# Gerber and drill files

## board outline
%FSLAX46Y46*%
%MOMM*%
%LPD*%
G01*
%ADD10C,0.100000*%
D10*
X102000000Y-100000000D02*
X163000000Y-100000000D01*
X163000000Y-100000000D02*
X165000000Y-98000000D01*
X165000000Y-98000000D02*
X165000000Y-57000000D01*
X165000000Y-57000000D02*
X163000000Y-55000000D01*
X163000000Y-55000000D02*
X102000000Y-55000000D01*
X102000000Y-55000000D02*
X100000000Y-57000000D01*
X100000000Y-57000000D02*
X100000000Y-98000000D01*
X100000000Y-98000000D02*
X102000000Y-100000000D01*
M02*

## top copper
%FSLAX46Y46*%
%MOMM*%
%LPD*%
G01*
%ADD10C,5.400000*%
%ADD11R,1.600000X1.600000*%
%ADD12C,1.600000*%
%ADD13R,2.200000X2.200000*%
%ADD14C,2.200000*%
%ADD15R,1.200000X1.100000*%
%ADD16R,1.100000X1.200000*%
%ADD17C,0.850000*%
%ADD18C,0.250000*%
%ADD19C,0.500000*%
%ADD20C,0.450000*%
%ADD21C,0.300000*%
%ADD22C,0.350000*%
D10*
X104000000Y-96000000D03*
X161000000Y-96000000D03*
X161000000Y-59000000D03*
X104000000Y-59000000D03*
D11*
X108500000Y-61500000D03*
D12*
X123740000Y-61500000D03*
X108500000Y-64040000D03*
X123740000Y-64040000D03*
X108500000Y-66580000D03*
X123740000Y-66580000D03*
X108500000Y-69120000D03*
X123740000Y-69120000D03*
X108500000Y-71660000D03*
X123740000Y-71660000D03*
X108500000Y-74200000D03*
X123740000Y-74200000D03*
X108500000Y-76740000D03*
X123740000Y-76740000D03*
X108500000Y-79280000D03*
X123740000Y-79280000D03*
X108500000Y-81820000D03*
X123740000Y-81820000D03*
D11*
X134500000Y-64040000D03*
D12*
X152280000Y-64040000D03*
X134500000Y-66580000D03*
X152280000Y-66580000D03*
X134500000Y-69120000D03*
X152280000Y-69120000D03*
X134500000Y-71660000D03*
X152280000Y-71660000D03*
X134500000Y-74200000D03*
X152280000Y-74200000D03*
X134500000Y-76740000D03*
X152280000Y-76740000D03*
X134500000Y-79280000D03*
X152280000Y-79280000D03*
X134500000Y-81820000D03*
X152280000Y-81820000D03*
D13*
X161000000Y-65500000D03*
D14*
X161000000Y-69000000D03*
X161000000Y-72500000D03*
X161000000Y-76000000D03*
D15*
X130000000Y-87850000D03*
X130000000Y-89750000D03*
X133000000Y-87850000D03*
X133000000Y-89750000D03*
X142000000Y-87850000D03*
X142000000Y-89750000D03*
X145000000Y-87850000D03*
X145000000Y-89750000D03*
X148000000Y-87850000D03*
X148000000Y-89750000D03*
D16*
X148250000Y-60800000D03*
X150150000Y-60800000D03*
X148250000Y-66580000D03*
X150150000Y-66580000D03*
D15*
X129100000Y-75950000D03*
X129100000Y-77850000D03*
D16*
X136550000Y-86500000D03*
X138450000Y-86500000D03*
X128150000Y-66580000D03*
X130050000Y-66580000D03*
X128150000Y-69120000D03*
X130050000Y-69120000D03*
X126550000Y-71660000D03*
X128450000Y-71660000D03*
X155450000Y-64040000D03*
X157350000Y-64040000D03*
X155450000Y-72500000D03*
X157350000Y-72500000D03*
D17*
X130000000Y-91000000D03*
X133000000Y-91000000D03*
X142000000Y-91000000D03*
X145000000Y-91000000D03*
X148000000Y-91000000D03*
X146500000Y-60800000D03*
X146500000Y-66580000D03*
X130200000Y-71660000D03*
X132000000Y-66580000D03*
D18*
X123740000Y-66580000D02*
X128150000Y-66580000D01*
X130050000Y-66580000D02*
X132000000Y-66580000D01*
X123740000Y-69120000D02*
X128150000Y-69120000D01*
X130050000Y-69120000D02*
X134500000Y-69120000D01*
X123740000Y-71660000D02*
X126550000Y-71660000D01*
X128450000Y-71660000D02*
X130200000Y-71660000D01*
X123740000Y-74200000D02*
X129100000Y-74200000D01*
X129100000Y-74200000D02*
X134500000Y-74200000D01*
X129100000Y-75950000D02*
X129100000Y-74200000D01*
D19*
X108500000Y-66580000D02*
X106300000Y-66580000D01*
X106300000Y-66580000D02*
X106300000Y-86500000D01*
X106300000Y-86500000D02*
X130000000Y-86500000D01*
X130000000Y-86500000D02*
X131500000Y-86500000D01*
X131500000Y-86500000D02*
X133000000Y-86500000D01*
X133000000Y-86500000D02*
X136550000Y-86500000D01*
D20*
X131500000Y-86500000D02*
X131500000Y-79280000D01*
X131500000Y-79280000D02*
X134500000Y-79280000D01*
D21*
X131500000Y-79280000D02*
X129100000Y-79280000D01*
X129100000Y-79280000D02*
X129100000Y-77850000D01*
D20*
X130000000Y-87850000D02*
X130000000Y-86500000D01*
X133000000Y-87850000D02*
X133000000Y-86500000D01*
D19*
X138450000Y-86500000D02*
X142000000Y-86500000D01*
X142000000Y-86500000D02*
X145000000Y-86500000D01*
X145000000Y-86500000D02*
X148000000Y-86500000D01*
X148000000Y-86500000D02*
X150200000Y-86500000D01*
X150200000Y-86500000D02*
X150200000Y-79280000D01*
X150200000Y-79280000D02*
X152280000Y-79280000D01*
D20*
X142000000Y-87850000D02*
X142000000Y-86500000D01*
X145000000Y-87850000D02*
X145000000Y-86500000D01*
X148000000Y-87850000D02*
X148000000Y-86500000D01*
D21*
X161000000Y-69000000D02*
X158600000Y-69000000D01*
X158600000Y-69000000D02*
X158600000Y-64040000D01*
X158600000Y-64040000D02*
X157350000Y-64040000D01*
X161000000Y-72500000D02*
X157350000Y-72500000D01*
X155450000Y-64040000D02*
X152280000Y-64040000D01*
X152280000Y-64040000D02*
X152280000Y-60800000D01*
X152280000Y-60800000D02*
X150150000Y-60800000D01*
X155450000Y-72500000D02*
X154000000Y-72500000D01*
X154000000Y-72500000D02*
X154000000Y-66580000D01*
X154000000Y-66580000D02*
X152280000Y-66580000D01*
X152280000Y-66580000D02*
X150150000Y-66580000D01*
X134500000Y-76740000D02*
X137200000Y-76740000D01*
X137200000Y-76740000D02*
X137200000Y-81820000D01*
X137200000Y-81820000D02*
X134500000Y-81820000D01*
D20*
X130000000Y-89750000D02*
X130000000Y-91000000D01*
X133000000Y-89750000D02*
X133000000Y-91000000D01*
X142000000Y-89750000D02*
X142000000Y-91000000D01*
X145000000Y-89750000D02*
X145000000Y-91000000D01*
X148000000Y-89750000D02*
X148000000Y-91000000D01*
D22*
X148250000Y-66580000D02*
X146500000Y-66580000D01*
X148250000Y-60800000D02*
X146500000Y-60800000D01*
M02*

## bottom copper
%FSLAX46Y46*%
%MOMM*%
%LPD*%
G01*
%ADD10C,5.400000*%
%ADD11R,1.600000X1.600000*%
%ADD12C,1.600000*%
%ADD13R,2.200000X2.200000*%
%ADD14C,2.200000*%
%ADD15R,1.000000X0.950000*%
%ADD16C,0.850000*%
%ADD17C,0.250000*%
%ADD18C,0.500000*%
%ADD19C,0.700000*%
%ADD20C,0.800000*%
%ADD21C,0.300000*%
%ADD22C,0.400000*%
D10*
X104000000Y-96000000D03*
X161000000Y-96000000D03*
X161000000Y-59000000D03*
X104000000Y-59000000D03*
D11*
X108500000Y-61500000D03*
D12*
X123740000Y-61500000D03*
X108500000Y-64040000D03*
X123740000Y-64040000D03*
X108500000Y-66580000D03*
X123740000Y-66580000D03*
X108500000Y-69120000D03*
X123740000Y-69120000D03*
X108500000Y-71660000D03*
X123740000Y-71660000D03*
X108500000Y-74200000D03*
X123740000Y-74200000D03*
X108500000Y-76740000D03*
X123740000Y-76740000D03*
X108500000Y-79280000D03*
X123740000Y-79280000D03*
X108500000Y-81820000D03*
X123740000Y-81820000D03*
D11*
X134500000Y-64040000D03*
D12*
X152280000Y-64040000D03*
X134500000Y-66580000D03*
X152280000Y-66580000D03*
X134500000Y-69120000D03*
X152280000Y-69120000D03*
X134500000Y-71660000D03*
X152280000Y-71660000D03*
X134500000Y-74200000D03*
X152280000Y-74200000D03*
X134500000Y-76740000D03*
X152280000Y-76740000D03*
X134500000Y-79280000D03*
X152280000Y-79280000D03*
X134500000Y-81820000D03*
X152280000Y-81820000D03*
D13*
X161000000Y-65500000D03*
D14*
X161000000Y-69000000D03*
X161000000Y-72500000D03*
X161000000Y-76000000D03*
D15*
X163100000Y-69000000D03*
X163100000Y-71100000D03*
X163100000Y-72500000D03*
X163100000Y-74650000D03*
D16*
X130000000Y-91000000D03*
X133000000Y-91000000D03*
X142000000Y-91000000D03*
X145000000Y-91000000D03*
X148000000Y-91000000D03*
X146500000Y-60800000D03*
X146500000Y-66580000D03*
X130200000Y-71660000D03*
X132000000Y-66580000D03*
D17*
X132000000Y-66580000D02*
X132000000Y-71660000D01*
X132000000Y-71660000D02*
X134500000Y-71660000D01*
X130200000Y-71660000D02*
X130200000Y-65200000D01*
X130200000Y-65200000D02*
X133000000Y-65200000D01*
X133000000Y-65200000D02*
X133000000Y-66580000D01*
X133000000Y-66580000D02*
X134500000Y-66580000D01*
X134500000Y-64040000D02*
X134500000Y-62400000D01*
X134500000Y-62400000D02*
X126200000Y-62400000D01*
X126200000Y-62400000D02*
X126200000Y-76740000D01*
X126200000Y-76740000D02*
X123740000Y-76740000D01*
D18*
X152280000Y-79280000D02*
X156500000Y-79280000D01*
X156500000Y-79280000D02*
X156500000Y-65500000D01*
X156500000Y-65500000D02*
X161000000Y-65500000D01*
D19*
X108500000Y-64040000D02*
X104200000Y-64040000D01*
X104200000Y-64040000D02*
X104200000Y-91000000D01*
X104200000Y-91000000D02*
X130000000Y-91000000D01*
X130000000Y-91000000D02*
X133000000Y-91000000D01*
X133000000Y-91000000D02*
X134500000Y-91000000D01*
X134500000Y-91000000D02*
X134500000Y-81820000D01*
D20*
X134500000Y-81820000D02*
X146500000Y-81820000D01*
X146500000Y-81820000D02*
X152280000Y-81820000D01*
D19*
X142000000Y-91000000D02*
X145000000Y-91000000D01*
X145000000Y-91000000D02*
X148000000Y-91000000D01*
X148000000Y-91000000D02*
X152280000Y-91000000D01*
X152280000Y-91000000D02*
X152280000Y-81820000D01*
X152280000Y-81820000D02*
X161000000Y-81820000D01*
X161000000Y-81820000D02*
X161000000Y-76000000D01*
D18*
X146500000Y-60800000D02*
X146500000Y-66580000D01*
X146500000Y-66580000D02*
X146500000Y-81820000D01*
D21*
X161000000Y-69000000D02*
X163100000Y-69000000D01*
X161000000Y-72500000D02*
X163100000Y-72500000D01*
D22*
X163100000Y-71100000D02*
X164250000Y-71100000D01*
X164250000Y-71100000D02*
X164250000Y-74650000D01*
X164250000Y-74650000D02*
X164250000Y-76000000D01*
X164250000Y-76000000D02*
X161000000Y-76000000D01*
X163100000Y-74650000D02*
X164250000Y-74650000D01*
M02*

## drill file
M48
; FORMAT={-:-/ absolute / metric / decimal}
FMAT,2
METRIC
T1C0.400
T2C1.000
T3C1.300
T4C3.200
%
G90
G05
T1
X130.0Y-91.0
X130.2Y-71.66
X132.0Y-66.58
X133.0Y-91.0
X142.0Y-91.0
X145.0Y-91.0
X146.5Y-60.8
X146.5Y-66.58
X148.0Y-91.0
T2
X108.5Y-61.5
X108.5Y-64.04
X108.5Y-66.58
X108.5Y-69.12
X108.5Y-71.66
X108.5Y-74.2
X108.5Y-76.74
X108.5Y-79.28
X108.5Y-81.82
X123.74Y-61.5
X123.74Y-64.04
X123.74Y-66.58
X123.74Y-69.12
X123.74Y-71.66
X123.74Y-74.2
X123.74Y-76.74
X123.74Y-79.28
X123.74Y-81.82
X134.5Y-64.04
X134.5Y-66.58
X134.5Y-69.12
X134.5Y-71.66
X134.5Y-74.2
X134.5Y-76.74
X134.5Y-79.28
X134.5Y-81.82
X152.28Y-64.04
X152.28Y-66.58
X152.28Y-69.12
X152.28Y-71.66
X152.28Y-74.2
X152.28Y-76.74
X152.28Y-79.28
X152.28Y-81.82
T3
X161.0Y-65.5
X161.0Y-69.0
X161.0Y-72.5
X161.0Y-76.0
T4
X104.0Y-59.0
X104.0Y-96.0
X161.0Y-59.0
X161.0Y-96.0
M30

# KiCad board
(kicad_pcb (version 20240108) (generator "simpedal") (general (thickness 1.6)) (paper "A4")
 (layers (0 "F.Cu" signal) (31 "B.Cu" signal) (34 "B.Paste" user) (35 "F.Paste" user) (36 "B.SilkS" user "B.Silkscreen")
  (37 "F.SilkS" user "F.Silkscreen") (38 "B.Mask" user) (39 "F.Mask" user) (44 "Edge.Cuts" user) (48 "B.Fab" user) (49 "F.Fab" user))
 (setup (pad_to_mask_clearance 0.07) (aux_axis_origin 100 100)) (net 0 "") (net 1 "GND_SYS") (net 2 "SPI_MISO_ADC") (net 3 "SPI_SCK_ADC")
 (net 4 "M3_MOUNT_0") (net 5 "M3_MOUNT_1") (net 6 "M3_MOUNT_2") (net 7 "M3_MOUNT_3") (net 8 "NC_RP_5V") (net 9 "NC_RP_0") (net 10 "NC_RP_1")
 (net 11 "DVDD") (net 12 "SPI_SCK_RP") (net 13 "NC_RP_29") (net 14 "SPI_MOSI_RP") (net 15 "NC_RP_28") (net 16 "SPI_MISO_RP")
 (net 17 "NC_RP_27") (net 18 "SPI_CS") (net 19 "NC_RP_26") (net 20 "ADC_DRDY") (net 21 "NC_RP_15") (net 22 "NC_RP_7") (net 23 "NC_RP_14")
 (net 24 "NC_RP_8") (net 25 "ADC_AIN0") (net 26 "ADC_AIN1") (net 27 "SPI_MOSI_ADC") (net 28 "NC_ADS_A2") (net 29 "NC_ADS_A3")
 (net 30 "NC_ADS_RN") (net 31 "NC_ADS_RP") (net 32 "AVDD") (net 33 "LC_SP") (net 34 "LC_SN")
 (via (at 130.0000 91.0000) (size 0.85) (drill 0.4) (layers "F.Cu" "B.Cu") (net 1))
 (via (at 133.0000 91.0000) (size 0.85) (drill 0.4) (layers "F.Cu" "B.Cu") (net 1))
 (via (at 142.0000 91.0000) (size 0.85) (drill 0.4) (layers "F.Cu" "B.Cu") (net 1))
 (via (at 145.0000 91.0000) (size 0.85) (drill 0.4) (layers "F.Cu" "B.Cu") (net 1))
 (via (at 148.0000 91.0000) (size 0.85) (drill 0.4) (layers "F.Cu" "B.Cu") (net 1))
 (via (at 146.5000 60.8000) (size 0.85) (drill 0.4) (layers "F.Cu" "B.Cu") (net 1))
 (via (at 146.5000 66.5800) (size 0.85) (drill 0.4) (layers "F.Cu" "B.Cu") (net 1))
 (via (at 130.2000 71.6600) (size 0.85) (drill 0.4) (layers "F.Cu" "B.Cu") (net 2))
 (via (at 132.0000 66.5800) (size 0.85) (drill 0.4) (layers "F.Cu" "B.Cu") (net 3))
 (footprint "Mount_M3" (layer "F.Cu") (at 104.0000 96.0000)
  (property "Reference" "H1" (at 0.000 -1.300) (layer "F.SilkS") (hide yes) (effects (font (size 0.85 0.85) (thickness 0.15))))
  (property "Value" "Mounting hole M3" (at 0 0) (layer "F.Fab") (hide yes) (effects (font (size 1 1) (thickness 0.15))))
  (pad "1" thru_hole circle (at 0.0000 0.0000) (size 5.4 5.4) (drill 3.2) (layers "*.Cu" "*.Mask") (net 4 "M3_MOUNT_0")))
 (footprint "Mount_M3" (layer "F.Cu") (at 161.0000 96.0000)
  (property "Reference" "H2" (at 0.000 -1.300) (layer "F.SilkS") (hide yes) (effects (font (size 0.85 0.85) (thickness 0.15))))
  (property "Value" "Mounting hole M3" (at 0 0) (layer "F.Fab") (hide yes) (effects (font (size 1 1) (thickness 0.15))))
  (pad "1" thru_hole circle (at 0.0000 0.0000) (size 5.4 5.4) (drill 3.2) (layers "*.Cu" "*.Mask") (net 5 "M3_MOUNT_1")))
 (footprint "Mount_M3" (layer "F.Cu") (at 161.0000 59.0000)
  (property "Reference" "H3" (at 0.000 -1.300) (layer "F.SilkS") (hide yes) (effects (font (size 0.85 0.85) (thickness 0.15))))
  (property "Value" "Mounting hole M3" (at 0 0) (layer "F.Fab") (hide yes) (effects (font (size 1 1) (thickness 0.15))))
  (pad "1" thru_hole circle (at 0.0000 0.0000) (size 5.4 5.4) (drill 3.2) (layers "*.Cu" "*.Mask") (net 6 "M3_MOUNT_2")))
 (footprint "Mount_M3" (layer "F.Cu") (at 104.0000 59.0000)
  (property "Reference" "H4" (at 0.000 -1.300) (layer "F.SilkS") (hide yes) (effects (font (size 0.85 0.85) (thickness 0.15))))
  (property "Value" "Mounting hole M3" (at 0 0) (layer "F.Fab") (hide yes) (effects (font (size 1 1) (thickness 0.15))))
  (pad "1" thru_hole circle (at 0.0000 0.0000) (size 5.4 5.4) (drill 3.2) (layers "*.Cu" "*.Mask") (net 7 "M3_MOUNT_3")))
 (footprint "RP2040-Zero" (layer "F.Cu") (at 116.1200 71.6600)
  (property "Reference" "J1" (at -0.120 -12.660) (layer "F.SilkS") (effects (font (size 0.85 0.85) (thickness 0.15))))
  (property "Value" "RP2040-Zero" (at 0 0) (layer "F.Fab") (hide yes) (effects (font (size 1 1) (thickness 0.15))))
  (pad "1" thru_hole rect (at -7.6200 -10.1600) (size 1.6 1.6) (drill 1) (layers "*.Cu" "*.Mask") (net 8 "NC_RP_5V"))
  (pad "2" thru_hole circle (at 7.6200 -10.1600) (size 1.6 1.6) (drill 1) (layers "*.Cu" "*.Mask") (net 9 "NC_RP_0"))
  (pad "3" thru_hole circle (at -7.6200 -7.6200) (size 1.6 1.6) (drill 1) (layers "*.Cu" "*.Mask") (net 1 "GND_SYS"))
  (pad "4" thru_hole circle (at 7.6200 -7.6200) (size 1.6 1.6) (drill 1) (layers "*.Cu" "*.Mask") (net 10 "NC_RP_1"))
  (pad "5" thru_hole circle (at -7.6200 -5.0800) (size 1.6 1.6) (drill 1) (layers "*.Cu" "*.Mask") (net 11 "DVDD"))
  (pad "6" thru_hole circle (at 7.6200 -5.0800) (size 1.6 1.6) (drill 1) (layers "*.Cu" "*.Mask") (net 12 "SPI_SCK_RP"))
  (pad "7" thru_hole circle (at -7.6200 -2.5400) (size 1.6 1.6) (drill 1) (layers "*.Cu" "*.Mask") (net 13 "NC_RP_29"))
  (pad "8" thru_hole circle (at 7.6200 -2.5400) (size 1.6 1.6) (drill 1) (layers "*.Cu" "*.Mask") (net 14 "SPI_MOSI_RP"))
  (pad "9" thru_hole circle (at -7.6200 0.0000) (size 1.6 1.6) (drill 1) (layers "*.Cu" "*.Mask") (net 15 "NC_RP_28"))
  (pad "10" thru_hole circle (at 7.6200 0.0000) (size 1.6 1.6) (drill 1) (layers "*.Cu" "*.Mask") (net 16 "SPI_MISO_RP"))
  (pad "11" thru_hole circle (at -7.6200 2.5400) (size 1.6 1.6) (drill 1) (layers "*.Cu" "*.Mask") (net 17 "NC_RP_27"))
  (pad "12" thru_hole circle (at 7.6200 2.5400) (size 1.6 1.6) (drill 1) (layers "*.Cu" "*.Mask") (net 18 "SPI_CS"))
  (pad "13" thru_hole circle (at -7.6200 5.0800) (size 1.6 1.6) (drill 1) (layers "*.Cu" "*.Mask") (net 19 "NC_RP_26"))
  (pad "14" thru_hole circle (at 7.6200 5.0800) (size 1.6 1.6) (drill 1) (layers "*.Cu" "*.Mask") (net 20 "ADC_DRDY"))
  (pad "15" thru_hole circle (at -7.6200 7.6200) (size 1.6 1.6) (drill 1) (layers "*.Cu" "*.Mask") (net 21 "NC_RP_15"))
  (pad "16" thru_hole circle (at 7.6200 7.6200) (size 1.6 1.6) (drill 1) (layers "*.Cu" "*.Mask") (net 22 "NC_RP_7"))
  (pad "17" thru_hole circle (at -7.6200 10.1600) (size 1.6 1.6) (drill 1) (layers "*.Cu" "*.Mask") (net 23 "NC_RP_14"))
  (pad "18" thru_hole circle (at 7.6200 10.1600) (size 1.6 1.6) (drill 1) (layers "*.Cu" "*.Mask") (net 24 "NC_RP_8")))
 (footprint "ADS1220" (layer "F.Cu") (at 143.3900 72.9300)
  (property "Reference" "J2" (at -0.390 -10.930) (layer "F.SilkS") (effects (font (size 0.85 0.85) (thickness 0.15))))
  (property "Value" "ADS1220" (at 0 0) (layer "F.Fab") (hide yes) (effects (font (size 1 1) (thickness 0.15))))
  (pad "1" thru_hole rect (at -8.8900 -8.8900) (size 1.6 1.6) (drill 1) (layers "*.Cu" "*.Mask") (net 20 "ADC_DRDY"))
  (pad "2" thru_hole circle (at 8.8900 -8.8900) (size 1.6 1.6) (drill 1) (layers "*.Cu" "*.Mask") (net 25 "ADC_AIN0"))
  (pad "3" thru_hole circle (at -8.8900 -6.3500) (size 1.6 1.6) (drill 1) (layers "*.Cu" "*.Mask") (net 2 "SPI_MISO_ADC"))
  (pad "4" thru_hole circle (at 8.8900 -6.3500) (size 1.6 1.6) (drill 1) (layers "*.Cu" "*.Mask") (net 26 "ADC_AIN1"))
  (pad "5" thru_hole circle (at -8.8900 -3.8100) (size 1.6 1.6) (drill 1) (layers "*.Cu" "*.Mask") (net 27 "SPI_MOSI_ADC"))
  (pad "6" thru_hole circle (at 8.8900 -3.8100) (size 1.6 1.6) (drill 1) (layers "*.Cu" "*.Mask") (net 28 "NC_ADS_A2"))
  (pad "7" thru_hole circle (at -8.8900 -1.2700) (size 1.6 1.6) (drill 1) (layers "*.Cu" "*.Mask") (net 3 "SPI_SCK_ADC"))
  (pad "8" thru_hole circle (at 8.8900 -1.2700) (size 1.6 1.6) (drill 1) (layers "*.Cu" "*.Mask") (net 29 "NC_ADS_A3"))
  (pad "9" thru_hole circle (at -8.8900 1.2700) (size 1.6 1.6) (drill 1) (layers "*.Cu" "*.Mask") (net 18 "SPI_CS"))
  (pad "10" thru_hole circle (at 8.8900 1.2700) (size 1.6 1.6) (drill 1) (layers "*.Cu" "*.Mask") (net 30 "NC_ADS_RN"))
  (pad "11" thru_hole circle (at -8.8900 3.8100) (size 1.6 1.6) (drill 1) (layers "*.Cu" "*.Mask") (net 1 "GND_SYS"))
  (pad "12" thru_hole circle (at 8.8900 3.8100) (size 1.6 1.6) (drill 1) (layers "*.Cu" "*.Mask") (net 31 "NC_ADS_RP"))
  (pad "13" thru_hole circle (at -8.8900 6.3500) (size 1.6 1.6) (drill 1) (layers "*.Cu" "*.Mask") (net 11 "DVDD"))
  (pad "14" thru_hole circle (at 8.8900 6.3500) (size 1.6 1.6) (drill 1) (layers "*.Cu" "*.Mask") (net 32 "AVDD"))
  (pad "15" thru_hole circle (at -8.8900 8.8900) (size 1.6 1.6) (drill 1) (layers "*.Cu" "*.Mask") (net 1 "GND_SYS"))
  (pad "16" thru_hole circle (at 8.8900 8.8900) (size 1.6 1.6) (drill 1) (layers "*.Cu" "*.Mask") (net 1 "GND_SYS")))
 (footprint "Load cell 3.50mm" (layer "F.Cu") (at 161.0000 70.7500)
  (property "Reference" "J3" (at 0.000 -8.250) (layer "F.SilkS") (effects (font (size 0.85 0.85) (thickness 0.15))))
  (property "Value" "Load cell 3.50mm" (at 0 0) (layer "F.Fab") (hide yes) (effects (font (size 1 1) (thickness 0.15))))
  (pad "1" thru_hole rect (at 0.0000 -5.2500) (size 2.2 2.2) (drill 1.3) (layers "*.Cu" "*.Mask") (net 32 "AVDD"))
  (pad "2" thru_hole circle (at 0.0000 -1.7500) (size 2.2 2.2) (drill 1.3) (layers "*.Cu" "*.Mask") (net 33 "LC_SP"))
  (pad "3" thru_hole circle (at 0.0000 1.7500) (size 2.2 2.2) (drill 1.3) (layers "*.Cu" "*.Mask") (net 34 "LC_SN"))
  (pad "4" thru_hole circle (at 0.0000 5.2500) (size 2.2 2.2) (drill 1.3) (layers "*.Cu" "*.Mask") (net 1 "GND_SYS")))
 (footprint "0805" (layer "F.Cu") (at 130.0000 88.8000)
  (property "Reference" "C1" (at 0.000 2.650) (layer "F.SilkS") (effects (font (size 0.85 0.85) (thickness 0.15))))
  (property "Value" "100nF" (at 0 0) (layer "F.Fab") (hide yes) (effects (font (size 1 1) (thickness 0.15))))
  (pad "2" smd rect (at 0.0000 -0.9500) (size 1.2 1.1) (layers "F.Cu" "F.Paste" "F.Mask") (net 11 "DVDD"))
  (pad "1" smd rect (at 0.0000 0.9500) (size 1.2 1.1) (layers "F.Cu" "F.Paste" "F.Mask") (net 1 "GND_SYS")))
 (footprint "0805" (layer "F.Cu") (at 133.0000 88.8000)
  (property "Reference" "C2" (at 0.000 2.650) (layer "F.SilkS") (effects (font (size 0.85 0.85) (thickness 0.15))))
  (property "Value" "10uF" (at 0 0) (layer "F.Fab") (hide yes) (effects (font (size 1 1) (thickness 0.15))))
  (pad "2" smd rect (at 0.0000 -0.9500) (size 1.2 1.1) (layers "F.Cu" "F.Paste" "F.Mask") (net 11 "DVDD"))
  (pad "1" smd rect (at 0.0000 0.9500) (size 1.2 1.1) (layers "F.Cu" "F.Paste" "F.Mask") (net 1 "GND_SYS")))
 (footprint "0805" (layer "F.Cu") (at 142.0000 88.8000)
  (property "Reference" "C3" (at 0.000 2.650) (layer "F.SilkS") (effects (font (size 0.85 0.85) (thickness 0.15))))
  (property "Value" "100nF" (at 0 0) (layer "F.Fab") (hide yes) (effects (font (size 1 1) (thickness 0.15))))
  (pad "2" smd rect (at 0.0000 -0.9500) (size 1.2 1.1) (layers "F.Cu" "F.Paste" "F.Mask") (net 32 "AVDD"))
  (pad "1" smd rect (at 0.0000 0.9500) (size 1.2 1.1) (layers "F.Cu" "F.Paste" "F.Mask") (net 1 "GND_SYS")))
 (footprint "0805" (layer "F.Cu") (at 145.0000 88.8000)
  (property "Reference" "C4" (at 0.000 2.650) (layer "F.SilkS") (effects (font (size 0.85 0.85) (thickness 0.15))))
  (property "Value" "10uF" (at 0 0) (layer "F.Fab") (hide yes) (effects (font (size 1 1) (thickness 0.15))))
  (pad "2" smd rect (at 0.0000 -0.9500) (size 1.2 1.1) (layers "F.Cu" "F.Paste" "F.Mask") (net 32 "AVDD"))
  (pad "1" smd rect (at 0.0000 0.9500) (size 1.2 1.1) (layers "F.Cu" "F.Paste" "F.Mask") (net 1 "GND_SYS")))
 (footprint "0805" (layer "F.Cu") (at 148.0000 88.8000)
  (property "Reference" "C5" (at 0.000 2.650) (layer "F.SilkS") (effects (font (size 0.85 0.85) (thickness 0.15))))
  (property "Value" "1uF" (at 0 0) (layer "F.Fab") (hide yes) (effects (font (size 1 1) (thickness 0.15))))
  (pad "2" smd rect (at 0.0000 -0.9500) (size 1.2 1.1) (layers "F.Cu" "F.Paste" "F.Mask") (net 32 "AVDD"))
  (pad "1" smd rect (at 0.0000 0.9500) (size 1.2 1.1) (layers "F.Cu" "F.Paste" "F.Mask") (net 1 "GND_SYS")))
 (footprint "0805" (layer "F.Cu") (at 149.2000 60.8000)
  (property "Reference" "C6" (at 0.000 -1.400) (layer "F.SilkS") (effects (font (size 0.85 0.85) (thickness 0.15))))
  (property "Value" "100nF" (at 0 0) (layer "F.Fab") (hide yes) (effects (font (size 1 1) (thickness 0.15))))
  (pad "1" smd rect (at -0.9500 0.0000) (size 1.1 1.2) (layers "F.Cu" "F.Paste" "F.Mask") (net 1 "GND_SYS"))
  (pad "2" smd rect (at 0.9500 0.0000) (size 1.1 1.2) (layers "F.Cu" "F.Paste" "F.Mask") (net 25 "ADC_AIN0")))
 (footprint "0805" (layer "F.Cu") (at 149.2000 66.5800)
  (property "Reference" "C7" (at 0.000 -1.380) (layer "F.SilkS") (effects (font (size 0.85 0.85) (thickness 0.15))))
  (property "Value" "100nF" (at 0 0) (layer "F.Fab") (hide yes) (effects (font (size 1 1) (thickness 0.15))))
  (pad "1" smd rect (at -0.9500 0.0000) (size 1.1 1.2) (layers "F.Cu" "F.Paste" "F.Mask") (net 1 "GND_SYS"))
  (pad "2" smd rect (at 0.9500 0.0000) (size 1.1 1.2) (layers "F.Cu" "F.Paste" "F.Mask") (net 26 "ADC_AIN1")))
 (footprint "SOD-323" (layer "B.Cu") (at 163.1000 70.0500)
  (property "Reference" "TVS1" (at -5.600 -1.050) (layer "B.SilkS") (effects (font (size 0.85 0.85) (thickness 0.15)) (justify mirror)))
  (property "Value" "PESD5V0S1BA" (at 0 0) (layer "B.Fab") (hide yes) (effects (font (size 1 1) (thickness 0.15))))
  (pad "1" smd rect (at 0.0000 -1.0500) (size 1 0.95) (layers "B.Cu" "B.Paste" "B.Mask") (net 33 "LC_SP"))
  (pad "2" smd rect (at 0.0000 1.0500) (size 1 0.95) (layers "B.Cu" "B.Paste" "B.Mask") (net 1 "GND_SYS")))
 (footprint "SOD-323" (layer "B.Cu") (at 163.1000 73.5750)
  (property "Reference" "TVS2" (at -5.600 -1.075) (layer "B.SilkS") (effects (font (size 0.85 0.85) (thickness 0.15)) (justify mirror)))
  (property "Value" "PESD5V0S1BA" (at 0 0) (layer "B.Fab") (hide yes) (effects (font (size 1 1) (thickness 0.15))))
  (pad "1" smd rect (at 0.0000 -1.0750) (size 1 0.95) (layers "B.Cu" "B.Paste" "B.Mask") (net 34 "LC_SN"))
  (pad "2" smd rect (at 0.0000 1.0750) (size 1 0.95) (layers "B.Cu" "B.Paste" "B.Mask") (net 1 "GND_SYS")))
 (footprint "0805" (layer "F.Cu") (at 129.1000 76.9000)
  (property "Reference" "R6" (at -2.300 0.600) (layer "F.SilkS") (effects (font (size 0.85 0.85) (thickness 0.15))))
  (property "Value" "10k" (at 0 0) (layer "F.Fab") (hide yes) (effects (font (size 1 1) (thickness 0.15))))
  (pad "2" smd rect (at 0.0000 -0.9500) (size 1.2 1.1) (layers "F.Cu" "F.Paste" "F.Mask") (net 18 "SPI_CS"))
  (pad "1" smd rect (at 0.0000 0.9500) (size 1.2 1.1) (layers "F.Cu" "F.Paste" "F.Mask") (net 11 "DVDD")))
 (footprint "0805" (layer "F.Cu") (at 137.5000 86.5000)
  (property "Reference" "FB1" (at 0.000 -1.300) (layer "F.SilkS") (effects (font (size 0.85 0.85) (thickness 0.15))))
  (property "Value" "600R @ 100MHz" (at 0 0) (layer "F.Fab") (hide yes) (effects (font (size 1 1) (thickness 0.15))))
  (pad "1" smd rect (at -0.9500 0.0000) (size 1.1 1.2) (layers "F.Cu" "F.Paste" "F.Mask") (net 11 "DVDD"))
  (pad "2" smd rect (at 0.9500 0.0000) (size 1.1 1.2) (layers "F.Cu" "F.Paste" "F.Mask") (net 32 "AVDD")))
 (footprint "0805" (layer "F.Cu") (at 129.1000 66.5800)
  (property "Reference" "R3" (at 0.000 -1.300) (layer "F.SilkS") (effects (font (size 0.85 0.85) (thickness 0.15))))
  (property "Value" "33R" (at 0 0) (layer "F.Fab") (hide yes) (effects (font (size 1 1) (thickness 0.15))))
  (pad "1" smd rect (at -0.9500 0.0000) (size 1.1 1.2) (layers "F.Cu" "F.Paste" "F.Mask") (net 12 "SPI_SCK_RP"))
  (pad "2" smd rect (at 0.9500 0.0000) (size 1.1 1.2) (layers "F.Cu" "F.Paste" "F.Mask") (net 3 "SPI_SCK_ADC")))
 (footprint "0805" (layer "F.Cu") (at 129.1000 69.1200)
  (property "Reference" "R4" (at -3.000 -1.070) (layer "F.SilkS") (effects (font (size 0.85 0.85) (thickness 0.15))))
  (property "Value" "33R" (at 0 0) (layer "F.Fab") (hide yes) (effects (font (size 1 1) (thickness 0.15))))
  (pad "1" smd rect (at -0.9500 0.0000) (size 1.1 1.2) (layers "F.Cu" "F.Paste" "F.Mask") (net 14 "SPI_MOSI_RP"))
  (pad "2" smd rect (at 0.9500 0.0000) (size 1.1 1.2) (layers "F.Cu" "F.Paste" "F.Mask") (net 27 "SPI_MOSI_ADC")))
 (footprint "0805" (layer "F.Cu") (at 127.5000 71.6600)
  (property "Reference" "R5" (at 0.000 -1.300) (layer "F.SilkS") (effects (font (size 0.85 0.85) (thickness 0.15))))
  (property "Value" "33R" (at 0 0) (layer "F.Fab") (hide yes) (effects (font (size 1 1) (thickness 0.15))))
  (pad "1" smd rect (at -0.9500 0.0000) (size 1.1 1.2) (layers "F.Cu" "F.Paste" "F.Mask") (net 16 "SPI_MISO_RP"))
  (pad "2" smd rect (at 0.9500 0.0000) (size 1.1 1.2) (layers "F.Cu" "F.Paste" "F.Mask") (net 2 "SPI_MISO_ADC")))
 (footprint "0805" (layer "F.Cu") (at 156.4000 64.0400)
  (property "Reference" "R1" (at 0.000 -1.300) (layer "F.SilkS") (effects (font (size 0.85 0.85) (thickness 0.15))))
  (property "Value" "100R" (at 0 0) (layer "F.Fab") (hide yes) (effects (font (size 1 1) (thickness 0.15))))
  (pad "1" smd rect (at -0.9500 0.0000) (size 1.1 1.2) (layers "F.Cu" "F.Paste" "F.Mask") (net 25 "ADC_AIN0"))
  (pad "2" smd rect (at 0.9500 0.0000) (size 1.1 1.2) (layers "F.Cu" "F.Paste" "F.Mask") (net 33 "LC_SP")))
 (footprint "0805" (layer "F.Cu") (at 156.4000 72.5000)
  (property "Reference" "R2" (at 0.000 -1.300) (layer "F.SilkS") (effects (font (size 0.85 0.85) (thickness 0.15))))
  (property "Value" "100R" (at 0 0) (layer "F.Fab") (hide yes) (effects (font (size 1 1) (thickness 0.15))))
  (pad "1" smd rect (at -0.9500 0.0000) (size 1.1 1.2) (layers "F.Cu" "F.Paste" "F.Mask") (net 26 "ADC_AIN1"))
  (pad "2" smd rect (at 0.9500 0.0000) (size 1.1 1.2) (layers "F.Cu" "F.Paste" "F.Mask") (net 34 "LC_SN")))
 (segment (start 123.7400 66.5800) (end 128.1500 66.5800) (width 0.25) (layer "F.Cu") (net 12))
 (segment (start 130.0500 66.5800) (end 132.0000 66.5800) (width 0.25) (layer "F.Cu") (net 3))
 (segment (start 132.0000 66.5800) (end 132.0000 71.6600) (width 0.25) (layer "B.Cu") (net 3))
 (segment (start 132.0000 71.6600) (end 134.5000 71.6600) (width 0.25) (layer "B.Cu") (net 3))
 (segment (start 123.7400 69.1200) (end 128.1500 69.1200) (width 0.25) (layer "F.Cu") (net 14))
 (segment (start 130.0500 69.1200) (end 134.5000 69.1200) (width 0.25) (layer "F.Cu") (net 27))
 (segment (start 123.7400 71.6600) (end 126.5500 71.6600) (width 0.25) (layer "F.Cu") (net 16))
 (segment (start 128.4500 71.6600) (end 130.2000 71.6600) (width 0.25) (layer "F.Cu") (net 2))
 (segment (start 130.2000 71.6600) (end 130.2000 65.2000) (width 0.25) (layer "B.Cu") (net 2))
 (segment (start 130.2000 65.2000) (end 133.0000 65.2000) (width 0.25) (layer "B.Cu") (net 2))
 (segment (start 133.0000 65.2000) (end 133.0000 66.5800) (width 0.25) (layer "B.Cu") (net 2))
 (segment (start 133.0000 66.5800) (end 134.5000 66.5800) (width 0.25) (layer "B.Cu") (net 2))
 (segment (start 123.7400 74.2000) (end 129.1000 74.2000) (width 0.25) (layer "F.Cu") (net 18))
 (segment (start 129.1000 74.2000) (end 134.5000 74.2000) (width 0.25) (layer "F.Cu") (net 18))
 (segment (start 129.1000 75.9500) (end 129.1000 74.2000) (width 0.25) (layer "F.Cu") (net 18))
 (segment (start 134.5000 64.0400) (end 134.5000 62.4000) (width 0.25) (layer "B.Cu") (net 20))
 (segment (start 134.5000 62.4000) (end 126.2000 62.4000) (width 0.25) (layer "B.Cu") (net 20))
 (segment (start 126.2000 62.4000) (end 126.2000 76.7400) (width 0.25) (layer "B.Cu") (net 20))
 (segment (start 126.2000 76.7400) (end 123.7400 76.7400) (width 0.25) (layer "B.Cu") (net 20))
 (segment (start 108.5000 66.5800) (end 106.3000 66.5800) (width 0.5) (layer "F.Cu") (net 11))
 (segment (start 106.3000 66.5800) (end 106.3000 86.5000) (width 0.5) (layer "F.Cu") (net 11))
 (segment (start 106.3000 86.5000) (end 130.0000 86.5000) (width 0.5) (layer "F.Cu") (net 11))
 (segment (start 130.0000 86.5000) (end 131.5000 86.5000) (width 0.5) (layer "F.Cu") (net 11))
 (segment (start 131.5000 86.5000) (end 133.0000 86.5000) (width 0.5) (layer "F.Cu") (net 11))
 (segment (start 133.0000 86.5000) (end 136.5500 86.5000) (width 0.5) (layer "F.Cu") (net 11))
 (segment (start 131.5000 86.5000) (end 131.5000 79.2800) (width 0.45) (layer "F.Cu") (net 11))
 (segment (start 131.5000 79.2800) (end 134.5000 79.2800) (width 0.45) (layer "F.Cu") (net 11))
 (segment (start 131.5000 79.2800) (end 129.1000 79.2800) (width 0.3) (layer "F.Cu") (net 11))
 (segment (start 129.1000 79.2800) (end 129.1000 77.8500) (width 0.3) (layer "F.Cu") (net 11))
 (segment (start 130.0000 87.8500) (end 130.0000 86.5000) (width 0.45) (layer "F.Cu") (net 11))
 (segment (start 133.0000 87.8500) (end 133.0000 86.5000) (width 0.45) (layer "F.Cu") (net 11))
 (segment (start 138.4500 86.5000) (end 142.0000 86.5000) (width 0.5) (layer "F.Cu") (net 32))
 (segment (start 142.0000 86.5000) (end 145.0000 86.5000) (width 0.5) (layer "F.Cu") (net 32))
 (segment (start 145.0000 86.5000) (end 148.0000 86.5000) (width 0.5) (layer "F.Cu") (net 32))
 (segment (start 148.0000 86.5000) (end 150.2000 86.5000) (width 0.5) (layer "F.Cu") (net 32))
 (segment (start 150.2000 86.5000) (end 150.2000 79.2800) (width 0.5) (layer "F.Cu") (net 32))
 (segment (start 150.2000 79.2800) (end 152.2800 79.2800) (width 0.5) (layer "F.Cu") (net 32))
 (segment (start 142.0000 87.8500) (end 142.0000 86.5000) (width 0.45) (layer "F.Cu") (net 32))
 (segment (start 145.0000 87.8500) (end 145.0000 86.5000) (width 0.45) (layer "F.Cu") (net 32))
 (segment (start 148.0000 87.8500) (end 148.0000 86.5000) (width 0.45) (layer "F.Cu") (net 32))
 (segment (start 152.2800 79.2800) (end 156.5000 79.2800) (width 0.5) (layer "B.Cu") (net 32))
 (segment (start 156.5000 79.2800) (end 156.5000 65.5000) (width 0.5) (layer "B.Cu") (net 32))
 (segment (start 156.5000 65.5000) (end 161.0000 65.5000) (width 0.5) (layer "B.Cu") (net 32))
 (segment (start 161.0000 69.0000) (end 158.6000 69.0000) (width 0.3) (layer "F.Cu") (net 33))
 (segment (start 158.6000 69.0000) (end 158.6000 64.0400) (width 0.3) (layer "F.Cu") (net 33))
 (segment (start 158.6000 64.0400) (end 157.3500 64.0400) (width 0.3) (layer "F.Cu") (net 33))
 (segment (start 161.0000 72.5000) (end 157.3500 72.5000) (width 0.3) (layer "F.Cu") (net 34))
 (segment (start 155.4500 64.0400) (end 152.2800 64.0400) (width 0.3) (layer "F.Cu") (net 25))
 (segment (start 152.2800 64.0400) (end 152.2800 60.8000) (width 0.3) (layer "F.Cu") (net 25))
 (segment (start 152.2800 60.8000) (end 150.1500 60.8000) (width 0.3) (layer "F.Cu") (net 25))
 (segment (start 155.4500 72.5000) (end 154.0000 72.5000) (width 0.3) (layer "F.Cu") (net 26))
 (segment (start 154.0000 72.5000) (end 154.0000 66.5800) (width 0.3) (layer "F.Cu") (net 26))
 (segment (start 154.0000 66.5800) (end 152.2800 66.5800) (width 0.3) (layer "F.Cu") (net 26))
 (segment (start 152.2800 66.5800) (end 150.1500 66.5800) (width 0.3) (layer "F.Cu") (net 26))
 (segment (start 108.5000 64.0400) (end 104.2000 64.0400) (width 0.7) (layer "B.Cu") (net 1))
 (segment (start 104.2000 64.0400) (end 104.2000 91.0000) (width 0.7) (layer "B.Cu") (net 1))
 (segment (start 104.2000 91.0000) (end 130.0000 91.0000) (width 0.7) (layer "B.Cu") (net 1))
 (segment (start 130.0000 91.0000) (end 133.0000 91.0000) (width 0.7) (layer "B.Cu") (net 1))
 (segment (start 133.0000 91.0000) (end 134.5000 91.0000) (width 0.7) (layer "B.Cu") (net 1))
 (segment (start 134.5000 91.0000) (end 134.5000 81.8200) (width 0.7) (layer "B.Cu") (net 1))
 (segment (start 134.5000 76.7400) (end 137.2000 76.7400) (width 0.3) (layer "F.Cu") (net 1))
 (segment (start 137.2000 76.7400) (end 137.2000 81.8200) (width 0.3) (layer "F.Cu") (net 1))
 (segment (start 137.2000 81.8200) (end 134.5000 81.8200) (width 0.3) (layer "F.Cu") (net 1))
 (segment (start 134.5000 81.8200) (end 146.5000 81.8200) (width 0.8) (layer "B.Cu") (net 1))
 (segment (start 146.5000 81.8200) (end 152.2800 81.8200) (width 0.8) (layer "B.Cu") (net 1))
 (segment (start 142.0000 91.0000) (end 145.0000 91.0000) (width 0.7) (layer "B.Cu") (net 1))
 (segment (start 145.0000 91.0000) (end 148.0000 91.0000) (width 0.7) (layer "B.Cu") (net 1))
 (segment (start 148.0000 91.0000) (end 152.2800 91.0000) (width 0.7) (layer "B.Cu") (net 1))
 (segment (start 152.2800 91.0000) (end 152.2800 81.8200) (width 0.7) (layer "B.Cu") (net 1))
 (segment (start 152.2800 81.8200) (end 161.0000 81.8200) (width 0.7) (layer "B.Cu") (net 1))
 (segment (start 161.0000 81.8200) (end 161.0000 76.0000) (width 0.7) (layer "B.Cu") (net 1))
 (segment (start 130.0000 89.7500) (end 130.0000 91.0000) (width 0.45) (layer "F.Cu") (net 1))
 (segment (start 133.0000 89.7500) (end 133.0000 91.0000) (width 0.45) (layer "F.Cu") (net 1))
 (segment (start 142.0000 89.7500) (end 142.0000 91.0000) (width 0.45) (layer "F.Cu") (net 1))
 (segment (start 145.0000 89.7500) (end 145.0000 91.0000) (width 0.45) (layer "F.Cu") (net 1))
 (segment (start 148.0000 89.7500) (end 148.0000 91.0000) (width 0.45) (layer "F.Cu") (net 1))
 (segment (start 148.2500 66.5800) (end 146.5000 66.5800) (width 0.35) (layer "F.Cu") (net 1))
 (segment (start 148.2500 60.8000) (end 146.5000 60.8000) (width 0.35) (layer "F.Cu") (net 1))
 (segment (start 146.5000 60.8000) (end 146.5000 66.5800) (width 0.5) (layer "B.Cu") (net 1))
 (segment (start 146.5000 66.5800) (end 146.5000 81.8200) (width 0.5) (layer "B.Cu") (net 1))
 (segment (start 161.0000 69.0000) (end 163.1000 69.0000) (width 0.3) (layer "B.Cu") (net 33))
 (segment (start 161.0000 72.5000) (end 163.1000 72.5000) (width 0.3) (layer "B.Cu") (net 34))
 (segment (start 163.1000 71.1000) (end 164.2500 71.1000) (width 0.4) (layer "B.Cu") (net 1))
 (segment (start 164.2500 71.1000) (end 164.2500 74.6500) (width 0.4) (layer "B.Cu") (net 1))
 (segment (start 164.2500 74.6500) (end 164.2500 76.0000) (width 0.4) (layer "B.Cu") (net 1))
 (segment (start 164.2500 76.0000) (end 161.0000 76.0000) (width 0.4) (layer "B.Cu") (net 1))
 (segment (start 163.1000 74.6500) (end 164.2500 74.6500) (width 0.4) (layer "B.Cu") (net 1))
 (gr_line (start 102.0000 100.0000) (end 163.0000 100.0000) (stroke (width .1) (type default)) (layer "Edge.Cuts"))
 (gr_line (start 163.0000 100.0000) (end 165.0000 98.0000) (stroke (width .1) (type default)) (layer "Edge.Cuts"))
 (gr_line (start 165.0000 98.0000) (end 165.0000 57.0000) (stroke (width .1) (type default)) (layer "Edge.Cuts"))
 (gr_line (start 165.0000 57.0000) (end 163.0000 55.0000) (stroke (width .1) (type default)) (layer "Edge.Cuts"))
 (gr_line (start 163.0000 55.0000) (end 102.0000 55.0000) (stroke (width .1) (type default)) (layer "Edge.Cuts"))
 (gr_line (start 102.0000 55.0000) (end 100.0000 57.0000) (stroke (width .1) (type default)) (layer "Edge.Cuts"))
 (gr_line (start 100.0000 57.0000) (end 100.0000 98.0000) (stroke (width .1) (type default)) (layer "Edge.Cuts"))
 (gr_line (start 100.0000 98.0000) (end 102.0000 100.0000) (stroke (width .1) (type default)) (layer "Edge.Cuts")))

